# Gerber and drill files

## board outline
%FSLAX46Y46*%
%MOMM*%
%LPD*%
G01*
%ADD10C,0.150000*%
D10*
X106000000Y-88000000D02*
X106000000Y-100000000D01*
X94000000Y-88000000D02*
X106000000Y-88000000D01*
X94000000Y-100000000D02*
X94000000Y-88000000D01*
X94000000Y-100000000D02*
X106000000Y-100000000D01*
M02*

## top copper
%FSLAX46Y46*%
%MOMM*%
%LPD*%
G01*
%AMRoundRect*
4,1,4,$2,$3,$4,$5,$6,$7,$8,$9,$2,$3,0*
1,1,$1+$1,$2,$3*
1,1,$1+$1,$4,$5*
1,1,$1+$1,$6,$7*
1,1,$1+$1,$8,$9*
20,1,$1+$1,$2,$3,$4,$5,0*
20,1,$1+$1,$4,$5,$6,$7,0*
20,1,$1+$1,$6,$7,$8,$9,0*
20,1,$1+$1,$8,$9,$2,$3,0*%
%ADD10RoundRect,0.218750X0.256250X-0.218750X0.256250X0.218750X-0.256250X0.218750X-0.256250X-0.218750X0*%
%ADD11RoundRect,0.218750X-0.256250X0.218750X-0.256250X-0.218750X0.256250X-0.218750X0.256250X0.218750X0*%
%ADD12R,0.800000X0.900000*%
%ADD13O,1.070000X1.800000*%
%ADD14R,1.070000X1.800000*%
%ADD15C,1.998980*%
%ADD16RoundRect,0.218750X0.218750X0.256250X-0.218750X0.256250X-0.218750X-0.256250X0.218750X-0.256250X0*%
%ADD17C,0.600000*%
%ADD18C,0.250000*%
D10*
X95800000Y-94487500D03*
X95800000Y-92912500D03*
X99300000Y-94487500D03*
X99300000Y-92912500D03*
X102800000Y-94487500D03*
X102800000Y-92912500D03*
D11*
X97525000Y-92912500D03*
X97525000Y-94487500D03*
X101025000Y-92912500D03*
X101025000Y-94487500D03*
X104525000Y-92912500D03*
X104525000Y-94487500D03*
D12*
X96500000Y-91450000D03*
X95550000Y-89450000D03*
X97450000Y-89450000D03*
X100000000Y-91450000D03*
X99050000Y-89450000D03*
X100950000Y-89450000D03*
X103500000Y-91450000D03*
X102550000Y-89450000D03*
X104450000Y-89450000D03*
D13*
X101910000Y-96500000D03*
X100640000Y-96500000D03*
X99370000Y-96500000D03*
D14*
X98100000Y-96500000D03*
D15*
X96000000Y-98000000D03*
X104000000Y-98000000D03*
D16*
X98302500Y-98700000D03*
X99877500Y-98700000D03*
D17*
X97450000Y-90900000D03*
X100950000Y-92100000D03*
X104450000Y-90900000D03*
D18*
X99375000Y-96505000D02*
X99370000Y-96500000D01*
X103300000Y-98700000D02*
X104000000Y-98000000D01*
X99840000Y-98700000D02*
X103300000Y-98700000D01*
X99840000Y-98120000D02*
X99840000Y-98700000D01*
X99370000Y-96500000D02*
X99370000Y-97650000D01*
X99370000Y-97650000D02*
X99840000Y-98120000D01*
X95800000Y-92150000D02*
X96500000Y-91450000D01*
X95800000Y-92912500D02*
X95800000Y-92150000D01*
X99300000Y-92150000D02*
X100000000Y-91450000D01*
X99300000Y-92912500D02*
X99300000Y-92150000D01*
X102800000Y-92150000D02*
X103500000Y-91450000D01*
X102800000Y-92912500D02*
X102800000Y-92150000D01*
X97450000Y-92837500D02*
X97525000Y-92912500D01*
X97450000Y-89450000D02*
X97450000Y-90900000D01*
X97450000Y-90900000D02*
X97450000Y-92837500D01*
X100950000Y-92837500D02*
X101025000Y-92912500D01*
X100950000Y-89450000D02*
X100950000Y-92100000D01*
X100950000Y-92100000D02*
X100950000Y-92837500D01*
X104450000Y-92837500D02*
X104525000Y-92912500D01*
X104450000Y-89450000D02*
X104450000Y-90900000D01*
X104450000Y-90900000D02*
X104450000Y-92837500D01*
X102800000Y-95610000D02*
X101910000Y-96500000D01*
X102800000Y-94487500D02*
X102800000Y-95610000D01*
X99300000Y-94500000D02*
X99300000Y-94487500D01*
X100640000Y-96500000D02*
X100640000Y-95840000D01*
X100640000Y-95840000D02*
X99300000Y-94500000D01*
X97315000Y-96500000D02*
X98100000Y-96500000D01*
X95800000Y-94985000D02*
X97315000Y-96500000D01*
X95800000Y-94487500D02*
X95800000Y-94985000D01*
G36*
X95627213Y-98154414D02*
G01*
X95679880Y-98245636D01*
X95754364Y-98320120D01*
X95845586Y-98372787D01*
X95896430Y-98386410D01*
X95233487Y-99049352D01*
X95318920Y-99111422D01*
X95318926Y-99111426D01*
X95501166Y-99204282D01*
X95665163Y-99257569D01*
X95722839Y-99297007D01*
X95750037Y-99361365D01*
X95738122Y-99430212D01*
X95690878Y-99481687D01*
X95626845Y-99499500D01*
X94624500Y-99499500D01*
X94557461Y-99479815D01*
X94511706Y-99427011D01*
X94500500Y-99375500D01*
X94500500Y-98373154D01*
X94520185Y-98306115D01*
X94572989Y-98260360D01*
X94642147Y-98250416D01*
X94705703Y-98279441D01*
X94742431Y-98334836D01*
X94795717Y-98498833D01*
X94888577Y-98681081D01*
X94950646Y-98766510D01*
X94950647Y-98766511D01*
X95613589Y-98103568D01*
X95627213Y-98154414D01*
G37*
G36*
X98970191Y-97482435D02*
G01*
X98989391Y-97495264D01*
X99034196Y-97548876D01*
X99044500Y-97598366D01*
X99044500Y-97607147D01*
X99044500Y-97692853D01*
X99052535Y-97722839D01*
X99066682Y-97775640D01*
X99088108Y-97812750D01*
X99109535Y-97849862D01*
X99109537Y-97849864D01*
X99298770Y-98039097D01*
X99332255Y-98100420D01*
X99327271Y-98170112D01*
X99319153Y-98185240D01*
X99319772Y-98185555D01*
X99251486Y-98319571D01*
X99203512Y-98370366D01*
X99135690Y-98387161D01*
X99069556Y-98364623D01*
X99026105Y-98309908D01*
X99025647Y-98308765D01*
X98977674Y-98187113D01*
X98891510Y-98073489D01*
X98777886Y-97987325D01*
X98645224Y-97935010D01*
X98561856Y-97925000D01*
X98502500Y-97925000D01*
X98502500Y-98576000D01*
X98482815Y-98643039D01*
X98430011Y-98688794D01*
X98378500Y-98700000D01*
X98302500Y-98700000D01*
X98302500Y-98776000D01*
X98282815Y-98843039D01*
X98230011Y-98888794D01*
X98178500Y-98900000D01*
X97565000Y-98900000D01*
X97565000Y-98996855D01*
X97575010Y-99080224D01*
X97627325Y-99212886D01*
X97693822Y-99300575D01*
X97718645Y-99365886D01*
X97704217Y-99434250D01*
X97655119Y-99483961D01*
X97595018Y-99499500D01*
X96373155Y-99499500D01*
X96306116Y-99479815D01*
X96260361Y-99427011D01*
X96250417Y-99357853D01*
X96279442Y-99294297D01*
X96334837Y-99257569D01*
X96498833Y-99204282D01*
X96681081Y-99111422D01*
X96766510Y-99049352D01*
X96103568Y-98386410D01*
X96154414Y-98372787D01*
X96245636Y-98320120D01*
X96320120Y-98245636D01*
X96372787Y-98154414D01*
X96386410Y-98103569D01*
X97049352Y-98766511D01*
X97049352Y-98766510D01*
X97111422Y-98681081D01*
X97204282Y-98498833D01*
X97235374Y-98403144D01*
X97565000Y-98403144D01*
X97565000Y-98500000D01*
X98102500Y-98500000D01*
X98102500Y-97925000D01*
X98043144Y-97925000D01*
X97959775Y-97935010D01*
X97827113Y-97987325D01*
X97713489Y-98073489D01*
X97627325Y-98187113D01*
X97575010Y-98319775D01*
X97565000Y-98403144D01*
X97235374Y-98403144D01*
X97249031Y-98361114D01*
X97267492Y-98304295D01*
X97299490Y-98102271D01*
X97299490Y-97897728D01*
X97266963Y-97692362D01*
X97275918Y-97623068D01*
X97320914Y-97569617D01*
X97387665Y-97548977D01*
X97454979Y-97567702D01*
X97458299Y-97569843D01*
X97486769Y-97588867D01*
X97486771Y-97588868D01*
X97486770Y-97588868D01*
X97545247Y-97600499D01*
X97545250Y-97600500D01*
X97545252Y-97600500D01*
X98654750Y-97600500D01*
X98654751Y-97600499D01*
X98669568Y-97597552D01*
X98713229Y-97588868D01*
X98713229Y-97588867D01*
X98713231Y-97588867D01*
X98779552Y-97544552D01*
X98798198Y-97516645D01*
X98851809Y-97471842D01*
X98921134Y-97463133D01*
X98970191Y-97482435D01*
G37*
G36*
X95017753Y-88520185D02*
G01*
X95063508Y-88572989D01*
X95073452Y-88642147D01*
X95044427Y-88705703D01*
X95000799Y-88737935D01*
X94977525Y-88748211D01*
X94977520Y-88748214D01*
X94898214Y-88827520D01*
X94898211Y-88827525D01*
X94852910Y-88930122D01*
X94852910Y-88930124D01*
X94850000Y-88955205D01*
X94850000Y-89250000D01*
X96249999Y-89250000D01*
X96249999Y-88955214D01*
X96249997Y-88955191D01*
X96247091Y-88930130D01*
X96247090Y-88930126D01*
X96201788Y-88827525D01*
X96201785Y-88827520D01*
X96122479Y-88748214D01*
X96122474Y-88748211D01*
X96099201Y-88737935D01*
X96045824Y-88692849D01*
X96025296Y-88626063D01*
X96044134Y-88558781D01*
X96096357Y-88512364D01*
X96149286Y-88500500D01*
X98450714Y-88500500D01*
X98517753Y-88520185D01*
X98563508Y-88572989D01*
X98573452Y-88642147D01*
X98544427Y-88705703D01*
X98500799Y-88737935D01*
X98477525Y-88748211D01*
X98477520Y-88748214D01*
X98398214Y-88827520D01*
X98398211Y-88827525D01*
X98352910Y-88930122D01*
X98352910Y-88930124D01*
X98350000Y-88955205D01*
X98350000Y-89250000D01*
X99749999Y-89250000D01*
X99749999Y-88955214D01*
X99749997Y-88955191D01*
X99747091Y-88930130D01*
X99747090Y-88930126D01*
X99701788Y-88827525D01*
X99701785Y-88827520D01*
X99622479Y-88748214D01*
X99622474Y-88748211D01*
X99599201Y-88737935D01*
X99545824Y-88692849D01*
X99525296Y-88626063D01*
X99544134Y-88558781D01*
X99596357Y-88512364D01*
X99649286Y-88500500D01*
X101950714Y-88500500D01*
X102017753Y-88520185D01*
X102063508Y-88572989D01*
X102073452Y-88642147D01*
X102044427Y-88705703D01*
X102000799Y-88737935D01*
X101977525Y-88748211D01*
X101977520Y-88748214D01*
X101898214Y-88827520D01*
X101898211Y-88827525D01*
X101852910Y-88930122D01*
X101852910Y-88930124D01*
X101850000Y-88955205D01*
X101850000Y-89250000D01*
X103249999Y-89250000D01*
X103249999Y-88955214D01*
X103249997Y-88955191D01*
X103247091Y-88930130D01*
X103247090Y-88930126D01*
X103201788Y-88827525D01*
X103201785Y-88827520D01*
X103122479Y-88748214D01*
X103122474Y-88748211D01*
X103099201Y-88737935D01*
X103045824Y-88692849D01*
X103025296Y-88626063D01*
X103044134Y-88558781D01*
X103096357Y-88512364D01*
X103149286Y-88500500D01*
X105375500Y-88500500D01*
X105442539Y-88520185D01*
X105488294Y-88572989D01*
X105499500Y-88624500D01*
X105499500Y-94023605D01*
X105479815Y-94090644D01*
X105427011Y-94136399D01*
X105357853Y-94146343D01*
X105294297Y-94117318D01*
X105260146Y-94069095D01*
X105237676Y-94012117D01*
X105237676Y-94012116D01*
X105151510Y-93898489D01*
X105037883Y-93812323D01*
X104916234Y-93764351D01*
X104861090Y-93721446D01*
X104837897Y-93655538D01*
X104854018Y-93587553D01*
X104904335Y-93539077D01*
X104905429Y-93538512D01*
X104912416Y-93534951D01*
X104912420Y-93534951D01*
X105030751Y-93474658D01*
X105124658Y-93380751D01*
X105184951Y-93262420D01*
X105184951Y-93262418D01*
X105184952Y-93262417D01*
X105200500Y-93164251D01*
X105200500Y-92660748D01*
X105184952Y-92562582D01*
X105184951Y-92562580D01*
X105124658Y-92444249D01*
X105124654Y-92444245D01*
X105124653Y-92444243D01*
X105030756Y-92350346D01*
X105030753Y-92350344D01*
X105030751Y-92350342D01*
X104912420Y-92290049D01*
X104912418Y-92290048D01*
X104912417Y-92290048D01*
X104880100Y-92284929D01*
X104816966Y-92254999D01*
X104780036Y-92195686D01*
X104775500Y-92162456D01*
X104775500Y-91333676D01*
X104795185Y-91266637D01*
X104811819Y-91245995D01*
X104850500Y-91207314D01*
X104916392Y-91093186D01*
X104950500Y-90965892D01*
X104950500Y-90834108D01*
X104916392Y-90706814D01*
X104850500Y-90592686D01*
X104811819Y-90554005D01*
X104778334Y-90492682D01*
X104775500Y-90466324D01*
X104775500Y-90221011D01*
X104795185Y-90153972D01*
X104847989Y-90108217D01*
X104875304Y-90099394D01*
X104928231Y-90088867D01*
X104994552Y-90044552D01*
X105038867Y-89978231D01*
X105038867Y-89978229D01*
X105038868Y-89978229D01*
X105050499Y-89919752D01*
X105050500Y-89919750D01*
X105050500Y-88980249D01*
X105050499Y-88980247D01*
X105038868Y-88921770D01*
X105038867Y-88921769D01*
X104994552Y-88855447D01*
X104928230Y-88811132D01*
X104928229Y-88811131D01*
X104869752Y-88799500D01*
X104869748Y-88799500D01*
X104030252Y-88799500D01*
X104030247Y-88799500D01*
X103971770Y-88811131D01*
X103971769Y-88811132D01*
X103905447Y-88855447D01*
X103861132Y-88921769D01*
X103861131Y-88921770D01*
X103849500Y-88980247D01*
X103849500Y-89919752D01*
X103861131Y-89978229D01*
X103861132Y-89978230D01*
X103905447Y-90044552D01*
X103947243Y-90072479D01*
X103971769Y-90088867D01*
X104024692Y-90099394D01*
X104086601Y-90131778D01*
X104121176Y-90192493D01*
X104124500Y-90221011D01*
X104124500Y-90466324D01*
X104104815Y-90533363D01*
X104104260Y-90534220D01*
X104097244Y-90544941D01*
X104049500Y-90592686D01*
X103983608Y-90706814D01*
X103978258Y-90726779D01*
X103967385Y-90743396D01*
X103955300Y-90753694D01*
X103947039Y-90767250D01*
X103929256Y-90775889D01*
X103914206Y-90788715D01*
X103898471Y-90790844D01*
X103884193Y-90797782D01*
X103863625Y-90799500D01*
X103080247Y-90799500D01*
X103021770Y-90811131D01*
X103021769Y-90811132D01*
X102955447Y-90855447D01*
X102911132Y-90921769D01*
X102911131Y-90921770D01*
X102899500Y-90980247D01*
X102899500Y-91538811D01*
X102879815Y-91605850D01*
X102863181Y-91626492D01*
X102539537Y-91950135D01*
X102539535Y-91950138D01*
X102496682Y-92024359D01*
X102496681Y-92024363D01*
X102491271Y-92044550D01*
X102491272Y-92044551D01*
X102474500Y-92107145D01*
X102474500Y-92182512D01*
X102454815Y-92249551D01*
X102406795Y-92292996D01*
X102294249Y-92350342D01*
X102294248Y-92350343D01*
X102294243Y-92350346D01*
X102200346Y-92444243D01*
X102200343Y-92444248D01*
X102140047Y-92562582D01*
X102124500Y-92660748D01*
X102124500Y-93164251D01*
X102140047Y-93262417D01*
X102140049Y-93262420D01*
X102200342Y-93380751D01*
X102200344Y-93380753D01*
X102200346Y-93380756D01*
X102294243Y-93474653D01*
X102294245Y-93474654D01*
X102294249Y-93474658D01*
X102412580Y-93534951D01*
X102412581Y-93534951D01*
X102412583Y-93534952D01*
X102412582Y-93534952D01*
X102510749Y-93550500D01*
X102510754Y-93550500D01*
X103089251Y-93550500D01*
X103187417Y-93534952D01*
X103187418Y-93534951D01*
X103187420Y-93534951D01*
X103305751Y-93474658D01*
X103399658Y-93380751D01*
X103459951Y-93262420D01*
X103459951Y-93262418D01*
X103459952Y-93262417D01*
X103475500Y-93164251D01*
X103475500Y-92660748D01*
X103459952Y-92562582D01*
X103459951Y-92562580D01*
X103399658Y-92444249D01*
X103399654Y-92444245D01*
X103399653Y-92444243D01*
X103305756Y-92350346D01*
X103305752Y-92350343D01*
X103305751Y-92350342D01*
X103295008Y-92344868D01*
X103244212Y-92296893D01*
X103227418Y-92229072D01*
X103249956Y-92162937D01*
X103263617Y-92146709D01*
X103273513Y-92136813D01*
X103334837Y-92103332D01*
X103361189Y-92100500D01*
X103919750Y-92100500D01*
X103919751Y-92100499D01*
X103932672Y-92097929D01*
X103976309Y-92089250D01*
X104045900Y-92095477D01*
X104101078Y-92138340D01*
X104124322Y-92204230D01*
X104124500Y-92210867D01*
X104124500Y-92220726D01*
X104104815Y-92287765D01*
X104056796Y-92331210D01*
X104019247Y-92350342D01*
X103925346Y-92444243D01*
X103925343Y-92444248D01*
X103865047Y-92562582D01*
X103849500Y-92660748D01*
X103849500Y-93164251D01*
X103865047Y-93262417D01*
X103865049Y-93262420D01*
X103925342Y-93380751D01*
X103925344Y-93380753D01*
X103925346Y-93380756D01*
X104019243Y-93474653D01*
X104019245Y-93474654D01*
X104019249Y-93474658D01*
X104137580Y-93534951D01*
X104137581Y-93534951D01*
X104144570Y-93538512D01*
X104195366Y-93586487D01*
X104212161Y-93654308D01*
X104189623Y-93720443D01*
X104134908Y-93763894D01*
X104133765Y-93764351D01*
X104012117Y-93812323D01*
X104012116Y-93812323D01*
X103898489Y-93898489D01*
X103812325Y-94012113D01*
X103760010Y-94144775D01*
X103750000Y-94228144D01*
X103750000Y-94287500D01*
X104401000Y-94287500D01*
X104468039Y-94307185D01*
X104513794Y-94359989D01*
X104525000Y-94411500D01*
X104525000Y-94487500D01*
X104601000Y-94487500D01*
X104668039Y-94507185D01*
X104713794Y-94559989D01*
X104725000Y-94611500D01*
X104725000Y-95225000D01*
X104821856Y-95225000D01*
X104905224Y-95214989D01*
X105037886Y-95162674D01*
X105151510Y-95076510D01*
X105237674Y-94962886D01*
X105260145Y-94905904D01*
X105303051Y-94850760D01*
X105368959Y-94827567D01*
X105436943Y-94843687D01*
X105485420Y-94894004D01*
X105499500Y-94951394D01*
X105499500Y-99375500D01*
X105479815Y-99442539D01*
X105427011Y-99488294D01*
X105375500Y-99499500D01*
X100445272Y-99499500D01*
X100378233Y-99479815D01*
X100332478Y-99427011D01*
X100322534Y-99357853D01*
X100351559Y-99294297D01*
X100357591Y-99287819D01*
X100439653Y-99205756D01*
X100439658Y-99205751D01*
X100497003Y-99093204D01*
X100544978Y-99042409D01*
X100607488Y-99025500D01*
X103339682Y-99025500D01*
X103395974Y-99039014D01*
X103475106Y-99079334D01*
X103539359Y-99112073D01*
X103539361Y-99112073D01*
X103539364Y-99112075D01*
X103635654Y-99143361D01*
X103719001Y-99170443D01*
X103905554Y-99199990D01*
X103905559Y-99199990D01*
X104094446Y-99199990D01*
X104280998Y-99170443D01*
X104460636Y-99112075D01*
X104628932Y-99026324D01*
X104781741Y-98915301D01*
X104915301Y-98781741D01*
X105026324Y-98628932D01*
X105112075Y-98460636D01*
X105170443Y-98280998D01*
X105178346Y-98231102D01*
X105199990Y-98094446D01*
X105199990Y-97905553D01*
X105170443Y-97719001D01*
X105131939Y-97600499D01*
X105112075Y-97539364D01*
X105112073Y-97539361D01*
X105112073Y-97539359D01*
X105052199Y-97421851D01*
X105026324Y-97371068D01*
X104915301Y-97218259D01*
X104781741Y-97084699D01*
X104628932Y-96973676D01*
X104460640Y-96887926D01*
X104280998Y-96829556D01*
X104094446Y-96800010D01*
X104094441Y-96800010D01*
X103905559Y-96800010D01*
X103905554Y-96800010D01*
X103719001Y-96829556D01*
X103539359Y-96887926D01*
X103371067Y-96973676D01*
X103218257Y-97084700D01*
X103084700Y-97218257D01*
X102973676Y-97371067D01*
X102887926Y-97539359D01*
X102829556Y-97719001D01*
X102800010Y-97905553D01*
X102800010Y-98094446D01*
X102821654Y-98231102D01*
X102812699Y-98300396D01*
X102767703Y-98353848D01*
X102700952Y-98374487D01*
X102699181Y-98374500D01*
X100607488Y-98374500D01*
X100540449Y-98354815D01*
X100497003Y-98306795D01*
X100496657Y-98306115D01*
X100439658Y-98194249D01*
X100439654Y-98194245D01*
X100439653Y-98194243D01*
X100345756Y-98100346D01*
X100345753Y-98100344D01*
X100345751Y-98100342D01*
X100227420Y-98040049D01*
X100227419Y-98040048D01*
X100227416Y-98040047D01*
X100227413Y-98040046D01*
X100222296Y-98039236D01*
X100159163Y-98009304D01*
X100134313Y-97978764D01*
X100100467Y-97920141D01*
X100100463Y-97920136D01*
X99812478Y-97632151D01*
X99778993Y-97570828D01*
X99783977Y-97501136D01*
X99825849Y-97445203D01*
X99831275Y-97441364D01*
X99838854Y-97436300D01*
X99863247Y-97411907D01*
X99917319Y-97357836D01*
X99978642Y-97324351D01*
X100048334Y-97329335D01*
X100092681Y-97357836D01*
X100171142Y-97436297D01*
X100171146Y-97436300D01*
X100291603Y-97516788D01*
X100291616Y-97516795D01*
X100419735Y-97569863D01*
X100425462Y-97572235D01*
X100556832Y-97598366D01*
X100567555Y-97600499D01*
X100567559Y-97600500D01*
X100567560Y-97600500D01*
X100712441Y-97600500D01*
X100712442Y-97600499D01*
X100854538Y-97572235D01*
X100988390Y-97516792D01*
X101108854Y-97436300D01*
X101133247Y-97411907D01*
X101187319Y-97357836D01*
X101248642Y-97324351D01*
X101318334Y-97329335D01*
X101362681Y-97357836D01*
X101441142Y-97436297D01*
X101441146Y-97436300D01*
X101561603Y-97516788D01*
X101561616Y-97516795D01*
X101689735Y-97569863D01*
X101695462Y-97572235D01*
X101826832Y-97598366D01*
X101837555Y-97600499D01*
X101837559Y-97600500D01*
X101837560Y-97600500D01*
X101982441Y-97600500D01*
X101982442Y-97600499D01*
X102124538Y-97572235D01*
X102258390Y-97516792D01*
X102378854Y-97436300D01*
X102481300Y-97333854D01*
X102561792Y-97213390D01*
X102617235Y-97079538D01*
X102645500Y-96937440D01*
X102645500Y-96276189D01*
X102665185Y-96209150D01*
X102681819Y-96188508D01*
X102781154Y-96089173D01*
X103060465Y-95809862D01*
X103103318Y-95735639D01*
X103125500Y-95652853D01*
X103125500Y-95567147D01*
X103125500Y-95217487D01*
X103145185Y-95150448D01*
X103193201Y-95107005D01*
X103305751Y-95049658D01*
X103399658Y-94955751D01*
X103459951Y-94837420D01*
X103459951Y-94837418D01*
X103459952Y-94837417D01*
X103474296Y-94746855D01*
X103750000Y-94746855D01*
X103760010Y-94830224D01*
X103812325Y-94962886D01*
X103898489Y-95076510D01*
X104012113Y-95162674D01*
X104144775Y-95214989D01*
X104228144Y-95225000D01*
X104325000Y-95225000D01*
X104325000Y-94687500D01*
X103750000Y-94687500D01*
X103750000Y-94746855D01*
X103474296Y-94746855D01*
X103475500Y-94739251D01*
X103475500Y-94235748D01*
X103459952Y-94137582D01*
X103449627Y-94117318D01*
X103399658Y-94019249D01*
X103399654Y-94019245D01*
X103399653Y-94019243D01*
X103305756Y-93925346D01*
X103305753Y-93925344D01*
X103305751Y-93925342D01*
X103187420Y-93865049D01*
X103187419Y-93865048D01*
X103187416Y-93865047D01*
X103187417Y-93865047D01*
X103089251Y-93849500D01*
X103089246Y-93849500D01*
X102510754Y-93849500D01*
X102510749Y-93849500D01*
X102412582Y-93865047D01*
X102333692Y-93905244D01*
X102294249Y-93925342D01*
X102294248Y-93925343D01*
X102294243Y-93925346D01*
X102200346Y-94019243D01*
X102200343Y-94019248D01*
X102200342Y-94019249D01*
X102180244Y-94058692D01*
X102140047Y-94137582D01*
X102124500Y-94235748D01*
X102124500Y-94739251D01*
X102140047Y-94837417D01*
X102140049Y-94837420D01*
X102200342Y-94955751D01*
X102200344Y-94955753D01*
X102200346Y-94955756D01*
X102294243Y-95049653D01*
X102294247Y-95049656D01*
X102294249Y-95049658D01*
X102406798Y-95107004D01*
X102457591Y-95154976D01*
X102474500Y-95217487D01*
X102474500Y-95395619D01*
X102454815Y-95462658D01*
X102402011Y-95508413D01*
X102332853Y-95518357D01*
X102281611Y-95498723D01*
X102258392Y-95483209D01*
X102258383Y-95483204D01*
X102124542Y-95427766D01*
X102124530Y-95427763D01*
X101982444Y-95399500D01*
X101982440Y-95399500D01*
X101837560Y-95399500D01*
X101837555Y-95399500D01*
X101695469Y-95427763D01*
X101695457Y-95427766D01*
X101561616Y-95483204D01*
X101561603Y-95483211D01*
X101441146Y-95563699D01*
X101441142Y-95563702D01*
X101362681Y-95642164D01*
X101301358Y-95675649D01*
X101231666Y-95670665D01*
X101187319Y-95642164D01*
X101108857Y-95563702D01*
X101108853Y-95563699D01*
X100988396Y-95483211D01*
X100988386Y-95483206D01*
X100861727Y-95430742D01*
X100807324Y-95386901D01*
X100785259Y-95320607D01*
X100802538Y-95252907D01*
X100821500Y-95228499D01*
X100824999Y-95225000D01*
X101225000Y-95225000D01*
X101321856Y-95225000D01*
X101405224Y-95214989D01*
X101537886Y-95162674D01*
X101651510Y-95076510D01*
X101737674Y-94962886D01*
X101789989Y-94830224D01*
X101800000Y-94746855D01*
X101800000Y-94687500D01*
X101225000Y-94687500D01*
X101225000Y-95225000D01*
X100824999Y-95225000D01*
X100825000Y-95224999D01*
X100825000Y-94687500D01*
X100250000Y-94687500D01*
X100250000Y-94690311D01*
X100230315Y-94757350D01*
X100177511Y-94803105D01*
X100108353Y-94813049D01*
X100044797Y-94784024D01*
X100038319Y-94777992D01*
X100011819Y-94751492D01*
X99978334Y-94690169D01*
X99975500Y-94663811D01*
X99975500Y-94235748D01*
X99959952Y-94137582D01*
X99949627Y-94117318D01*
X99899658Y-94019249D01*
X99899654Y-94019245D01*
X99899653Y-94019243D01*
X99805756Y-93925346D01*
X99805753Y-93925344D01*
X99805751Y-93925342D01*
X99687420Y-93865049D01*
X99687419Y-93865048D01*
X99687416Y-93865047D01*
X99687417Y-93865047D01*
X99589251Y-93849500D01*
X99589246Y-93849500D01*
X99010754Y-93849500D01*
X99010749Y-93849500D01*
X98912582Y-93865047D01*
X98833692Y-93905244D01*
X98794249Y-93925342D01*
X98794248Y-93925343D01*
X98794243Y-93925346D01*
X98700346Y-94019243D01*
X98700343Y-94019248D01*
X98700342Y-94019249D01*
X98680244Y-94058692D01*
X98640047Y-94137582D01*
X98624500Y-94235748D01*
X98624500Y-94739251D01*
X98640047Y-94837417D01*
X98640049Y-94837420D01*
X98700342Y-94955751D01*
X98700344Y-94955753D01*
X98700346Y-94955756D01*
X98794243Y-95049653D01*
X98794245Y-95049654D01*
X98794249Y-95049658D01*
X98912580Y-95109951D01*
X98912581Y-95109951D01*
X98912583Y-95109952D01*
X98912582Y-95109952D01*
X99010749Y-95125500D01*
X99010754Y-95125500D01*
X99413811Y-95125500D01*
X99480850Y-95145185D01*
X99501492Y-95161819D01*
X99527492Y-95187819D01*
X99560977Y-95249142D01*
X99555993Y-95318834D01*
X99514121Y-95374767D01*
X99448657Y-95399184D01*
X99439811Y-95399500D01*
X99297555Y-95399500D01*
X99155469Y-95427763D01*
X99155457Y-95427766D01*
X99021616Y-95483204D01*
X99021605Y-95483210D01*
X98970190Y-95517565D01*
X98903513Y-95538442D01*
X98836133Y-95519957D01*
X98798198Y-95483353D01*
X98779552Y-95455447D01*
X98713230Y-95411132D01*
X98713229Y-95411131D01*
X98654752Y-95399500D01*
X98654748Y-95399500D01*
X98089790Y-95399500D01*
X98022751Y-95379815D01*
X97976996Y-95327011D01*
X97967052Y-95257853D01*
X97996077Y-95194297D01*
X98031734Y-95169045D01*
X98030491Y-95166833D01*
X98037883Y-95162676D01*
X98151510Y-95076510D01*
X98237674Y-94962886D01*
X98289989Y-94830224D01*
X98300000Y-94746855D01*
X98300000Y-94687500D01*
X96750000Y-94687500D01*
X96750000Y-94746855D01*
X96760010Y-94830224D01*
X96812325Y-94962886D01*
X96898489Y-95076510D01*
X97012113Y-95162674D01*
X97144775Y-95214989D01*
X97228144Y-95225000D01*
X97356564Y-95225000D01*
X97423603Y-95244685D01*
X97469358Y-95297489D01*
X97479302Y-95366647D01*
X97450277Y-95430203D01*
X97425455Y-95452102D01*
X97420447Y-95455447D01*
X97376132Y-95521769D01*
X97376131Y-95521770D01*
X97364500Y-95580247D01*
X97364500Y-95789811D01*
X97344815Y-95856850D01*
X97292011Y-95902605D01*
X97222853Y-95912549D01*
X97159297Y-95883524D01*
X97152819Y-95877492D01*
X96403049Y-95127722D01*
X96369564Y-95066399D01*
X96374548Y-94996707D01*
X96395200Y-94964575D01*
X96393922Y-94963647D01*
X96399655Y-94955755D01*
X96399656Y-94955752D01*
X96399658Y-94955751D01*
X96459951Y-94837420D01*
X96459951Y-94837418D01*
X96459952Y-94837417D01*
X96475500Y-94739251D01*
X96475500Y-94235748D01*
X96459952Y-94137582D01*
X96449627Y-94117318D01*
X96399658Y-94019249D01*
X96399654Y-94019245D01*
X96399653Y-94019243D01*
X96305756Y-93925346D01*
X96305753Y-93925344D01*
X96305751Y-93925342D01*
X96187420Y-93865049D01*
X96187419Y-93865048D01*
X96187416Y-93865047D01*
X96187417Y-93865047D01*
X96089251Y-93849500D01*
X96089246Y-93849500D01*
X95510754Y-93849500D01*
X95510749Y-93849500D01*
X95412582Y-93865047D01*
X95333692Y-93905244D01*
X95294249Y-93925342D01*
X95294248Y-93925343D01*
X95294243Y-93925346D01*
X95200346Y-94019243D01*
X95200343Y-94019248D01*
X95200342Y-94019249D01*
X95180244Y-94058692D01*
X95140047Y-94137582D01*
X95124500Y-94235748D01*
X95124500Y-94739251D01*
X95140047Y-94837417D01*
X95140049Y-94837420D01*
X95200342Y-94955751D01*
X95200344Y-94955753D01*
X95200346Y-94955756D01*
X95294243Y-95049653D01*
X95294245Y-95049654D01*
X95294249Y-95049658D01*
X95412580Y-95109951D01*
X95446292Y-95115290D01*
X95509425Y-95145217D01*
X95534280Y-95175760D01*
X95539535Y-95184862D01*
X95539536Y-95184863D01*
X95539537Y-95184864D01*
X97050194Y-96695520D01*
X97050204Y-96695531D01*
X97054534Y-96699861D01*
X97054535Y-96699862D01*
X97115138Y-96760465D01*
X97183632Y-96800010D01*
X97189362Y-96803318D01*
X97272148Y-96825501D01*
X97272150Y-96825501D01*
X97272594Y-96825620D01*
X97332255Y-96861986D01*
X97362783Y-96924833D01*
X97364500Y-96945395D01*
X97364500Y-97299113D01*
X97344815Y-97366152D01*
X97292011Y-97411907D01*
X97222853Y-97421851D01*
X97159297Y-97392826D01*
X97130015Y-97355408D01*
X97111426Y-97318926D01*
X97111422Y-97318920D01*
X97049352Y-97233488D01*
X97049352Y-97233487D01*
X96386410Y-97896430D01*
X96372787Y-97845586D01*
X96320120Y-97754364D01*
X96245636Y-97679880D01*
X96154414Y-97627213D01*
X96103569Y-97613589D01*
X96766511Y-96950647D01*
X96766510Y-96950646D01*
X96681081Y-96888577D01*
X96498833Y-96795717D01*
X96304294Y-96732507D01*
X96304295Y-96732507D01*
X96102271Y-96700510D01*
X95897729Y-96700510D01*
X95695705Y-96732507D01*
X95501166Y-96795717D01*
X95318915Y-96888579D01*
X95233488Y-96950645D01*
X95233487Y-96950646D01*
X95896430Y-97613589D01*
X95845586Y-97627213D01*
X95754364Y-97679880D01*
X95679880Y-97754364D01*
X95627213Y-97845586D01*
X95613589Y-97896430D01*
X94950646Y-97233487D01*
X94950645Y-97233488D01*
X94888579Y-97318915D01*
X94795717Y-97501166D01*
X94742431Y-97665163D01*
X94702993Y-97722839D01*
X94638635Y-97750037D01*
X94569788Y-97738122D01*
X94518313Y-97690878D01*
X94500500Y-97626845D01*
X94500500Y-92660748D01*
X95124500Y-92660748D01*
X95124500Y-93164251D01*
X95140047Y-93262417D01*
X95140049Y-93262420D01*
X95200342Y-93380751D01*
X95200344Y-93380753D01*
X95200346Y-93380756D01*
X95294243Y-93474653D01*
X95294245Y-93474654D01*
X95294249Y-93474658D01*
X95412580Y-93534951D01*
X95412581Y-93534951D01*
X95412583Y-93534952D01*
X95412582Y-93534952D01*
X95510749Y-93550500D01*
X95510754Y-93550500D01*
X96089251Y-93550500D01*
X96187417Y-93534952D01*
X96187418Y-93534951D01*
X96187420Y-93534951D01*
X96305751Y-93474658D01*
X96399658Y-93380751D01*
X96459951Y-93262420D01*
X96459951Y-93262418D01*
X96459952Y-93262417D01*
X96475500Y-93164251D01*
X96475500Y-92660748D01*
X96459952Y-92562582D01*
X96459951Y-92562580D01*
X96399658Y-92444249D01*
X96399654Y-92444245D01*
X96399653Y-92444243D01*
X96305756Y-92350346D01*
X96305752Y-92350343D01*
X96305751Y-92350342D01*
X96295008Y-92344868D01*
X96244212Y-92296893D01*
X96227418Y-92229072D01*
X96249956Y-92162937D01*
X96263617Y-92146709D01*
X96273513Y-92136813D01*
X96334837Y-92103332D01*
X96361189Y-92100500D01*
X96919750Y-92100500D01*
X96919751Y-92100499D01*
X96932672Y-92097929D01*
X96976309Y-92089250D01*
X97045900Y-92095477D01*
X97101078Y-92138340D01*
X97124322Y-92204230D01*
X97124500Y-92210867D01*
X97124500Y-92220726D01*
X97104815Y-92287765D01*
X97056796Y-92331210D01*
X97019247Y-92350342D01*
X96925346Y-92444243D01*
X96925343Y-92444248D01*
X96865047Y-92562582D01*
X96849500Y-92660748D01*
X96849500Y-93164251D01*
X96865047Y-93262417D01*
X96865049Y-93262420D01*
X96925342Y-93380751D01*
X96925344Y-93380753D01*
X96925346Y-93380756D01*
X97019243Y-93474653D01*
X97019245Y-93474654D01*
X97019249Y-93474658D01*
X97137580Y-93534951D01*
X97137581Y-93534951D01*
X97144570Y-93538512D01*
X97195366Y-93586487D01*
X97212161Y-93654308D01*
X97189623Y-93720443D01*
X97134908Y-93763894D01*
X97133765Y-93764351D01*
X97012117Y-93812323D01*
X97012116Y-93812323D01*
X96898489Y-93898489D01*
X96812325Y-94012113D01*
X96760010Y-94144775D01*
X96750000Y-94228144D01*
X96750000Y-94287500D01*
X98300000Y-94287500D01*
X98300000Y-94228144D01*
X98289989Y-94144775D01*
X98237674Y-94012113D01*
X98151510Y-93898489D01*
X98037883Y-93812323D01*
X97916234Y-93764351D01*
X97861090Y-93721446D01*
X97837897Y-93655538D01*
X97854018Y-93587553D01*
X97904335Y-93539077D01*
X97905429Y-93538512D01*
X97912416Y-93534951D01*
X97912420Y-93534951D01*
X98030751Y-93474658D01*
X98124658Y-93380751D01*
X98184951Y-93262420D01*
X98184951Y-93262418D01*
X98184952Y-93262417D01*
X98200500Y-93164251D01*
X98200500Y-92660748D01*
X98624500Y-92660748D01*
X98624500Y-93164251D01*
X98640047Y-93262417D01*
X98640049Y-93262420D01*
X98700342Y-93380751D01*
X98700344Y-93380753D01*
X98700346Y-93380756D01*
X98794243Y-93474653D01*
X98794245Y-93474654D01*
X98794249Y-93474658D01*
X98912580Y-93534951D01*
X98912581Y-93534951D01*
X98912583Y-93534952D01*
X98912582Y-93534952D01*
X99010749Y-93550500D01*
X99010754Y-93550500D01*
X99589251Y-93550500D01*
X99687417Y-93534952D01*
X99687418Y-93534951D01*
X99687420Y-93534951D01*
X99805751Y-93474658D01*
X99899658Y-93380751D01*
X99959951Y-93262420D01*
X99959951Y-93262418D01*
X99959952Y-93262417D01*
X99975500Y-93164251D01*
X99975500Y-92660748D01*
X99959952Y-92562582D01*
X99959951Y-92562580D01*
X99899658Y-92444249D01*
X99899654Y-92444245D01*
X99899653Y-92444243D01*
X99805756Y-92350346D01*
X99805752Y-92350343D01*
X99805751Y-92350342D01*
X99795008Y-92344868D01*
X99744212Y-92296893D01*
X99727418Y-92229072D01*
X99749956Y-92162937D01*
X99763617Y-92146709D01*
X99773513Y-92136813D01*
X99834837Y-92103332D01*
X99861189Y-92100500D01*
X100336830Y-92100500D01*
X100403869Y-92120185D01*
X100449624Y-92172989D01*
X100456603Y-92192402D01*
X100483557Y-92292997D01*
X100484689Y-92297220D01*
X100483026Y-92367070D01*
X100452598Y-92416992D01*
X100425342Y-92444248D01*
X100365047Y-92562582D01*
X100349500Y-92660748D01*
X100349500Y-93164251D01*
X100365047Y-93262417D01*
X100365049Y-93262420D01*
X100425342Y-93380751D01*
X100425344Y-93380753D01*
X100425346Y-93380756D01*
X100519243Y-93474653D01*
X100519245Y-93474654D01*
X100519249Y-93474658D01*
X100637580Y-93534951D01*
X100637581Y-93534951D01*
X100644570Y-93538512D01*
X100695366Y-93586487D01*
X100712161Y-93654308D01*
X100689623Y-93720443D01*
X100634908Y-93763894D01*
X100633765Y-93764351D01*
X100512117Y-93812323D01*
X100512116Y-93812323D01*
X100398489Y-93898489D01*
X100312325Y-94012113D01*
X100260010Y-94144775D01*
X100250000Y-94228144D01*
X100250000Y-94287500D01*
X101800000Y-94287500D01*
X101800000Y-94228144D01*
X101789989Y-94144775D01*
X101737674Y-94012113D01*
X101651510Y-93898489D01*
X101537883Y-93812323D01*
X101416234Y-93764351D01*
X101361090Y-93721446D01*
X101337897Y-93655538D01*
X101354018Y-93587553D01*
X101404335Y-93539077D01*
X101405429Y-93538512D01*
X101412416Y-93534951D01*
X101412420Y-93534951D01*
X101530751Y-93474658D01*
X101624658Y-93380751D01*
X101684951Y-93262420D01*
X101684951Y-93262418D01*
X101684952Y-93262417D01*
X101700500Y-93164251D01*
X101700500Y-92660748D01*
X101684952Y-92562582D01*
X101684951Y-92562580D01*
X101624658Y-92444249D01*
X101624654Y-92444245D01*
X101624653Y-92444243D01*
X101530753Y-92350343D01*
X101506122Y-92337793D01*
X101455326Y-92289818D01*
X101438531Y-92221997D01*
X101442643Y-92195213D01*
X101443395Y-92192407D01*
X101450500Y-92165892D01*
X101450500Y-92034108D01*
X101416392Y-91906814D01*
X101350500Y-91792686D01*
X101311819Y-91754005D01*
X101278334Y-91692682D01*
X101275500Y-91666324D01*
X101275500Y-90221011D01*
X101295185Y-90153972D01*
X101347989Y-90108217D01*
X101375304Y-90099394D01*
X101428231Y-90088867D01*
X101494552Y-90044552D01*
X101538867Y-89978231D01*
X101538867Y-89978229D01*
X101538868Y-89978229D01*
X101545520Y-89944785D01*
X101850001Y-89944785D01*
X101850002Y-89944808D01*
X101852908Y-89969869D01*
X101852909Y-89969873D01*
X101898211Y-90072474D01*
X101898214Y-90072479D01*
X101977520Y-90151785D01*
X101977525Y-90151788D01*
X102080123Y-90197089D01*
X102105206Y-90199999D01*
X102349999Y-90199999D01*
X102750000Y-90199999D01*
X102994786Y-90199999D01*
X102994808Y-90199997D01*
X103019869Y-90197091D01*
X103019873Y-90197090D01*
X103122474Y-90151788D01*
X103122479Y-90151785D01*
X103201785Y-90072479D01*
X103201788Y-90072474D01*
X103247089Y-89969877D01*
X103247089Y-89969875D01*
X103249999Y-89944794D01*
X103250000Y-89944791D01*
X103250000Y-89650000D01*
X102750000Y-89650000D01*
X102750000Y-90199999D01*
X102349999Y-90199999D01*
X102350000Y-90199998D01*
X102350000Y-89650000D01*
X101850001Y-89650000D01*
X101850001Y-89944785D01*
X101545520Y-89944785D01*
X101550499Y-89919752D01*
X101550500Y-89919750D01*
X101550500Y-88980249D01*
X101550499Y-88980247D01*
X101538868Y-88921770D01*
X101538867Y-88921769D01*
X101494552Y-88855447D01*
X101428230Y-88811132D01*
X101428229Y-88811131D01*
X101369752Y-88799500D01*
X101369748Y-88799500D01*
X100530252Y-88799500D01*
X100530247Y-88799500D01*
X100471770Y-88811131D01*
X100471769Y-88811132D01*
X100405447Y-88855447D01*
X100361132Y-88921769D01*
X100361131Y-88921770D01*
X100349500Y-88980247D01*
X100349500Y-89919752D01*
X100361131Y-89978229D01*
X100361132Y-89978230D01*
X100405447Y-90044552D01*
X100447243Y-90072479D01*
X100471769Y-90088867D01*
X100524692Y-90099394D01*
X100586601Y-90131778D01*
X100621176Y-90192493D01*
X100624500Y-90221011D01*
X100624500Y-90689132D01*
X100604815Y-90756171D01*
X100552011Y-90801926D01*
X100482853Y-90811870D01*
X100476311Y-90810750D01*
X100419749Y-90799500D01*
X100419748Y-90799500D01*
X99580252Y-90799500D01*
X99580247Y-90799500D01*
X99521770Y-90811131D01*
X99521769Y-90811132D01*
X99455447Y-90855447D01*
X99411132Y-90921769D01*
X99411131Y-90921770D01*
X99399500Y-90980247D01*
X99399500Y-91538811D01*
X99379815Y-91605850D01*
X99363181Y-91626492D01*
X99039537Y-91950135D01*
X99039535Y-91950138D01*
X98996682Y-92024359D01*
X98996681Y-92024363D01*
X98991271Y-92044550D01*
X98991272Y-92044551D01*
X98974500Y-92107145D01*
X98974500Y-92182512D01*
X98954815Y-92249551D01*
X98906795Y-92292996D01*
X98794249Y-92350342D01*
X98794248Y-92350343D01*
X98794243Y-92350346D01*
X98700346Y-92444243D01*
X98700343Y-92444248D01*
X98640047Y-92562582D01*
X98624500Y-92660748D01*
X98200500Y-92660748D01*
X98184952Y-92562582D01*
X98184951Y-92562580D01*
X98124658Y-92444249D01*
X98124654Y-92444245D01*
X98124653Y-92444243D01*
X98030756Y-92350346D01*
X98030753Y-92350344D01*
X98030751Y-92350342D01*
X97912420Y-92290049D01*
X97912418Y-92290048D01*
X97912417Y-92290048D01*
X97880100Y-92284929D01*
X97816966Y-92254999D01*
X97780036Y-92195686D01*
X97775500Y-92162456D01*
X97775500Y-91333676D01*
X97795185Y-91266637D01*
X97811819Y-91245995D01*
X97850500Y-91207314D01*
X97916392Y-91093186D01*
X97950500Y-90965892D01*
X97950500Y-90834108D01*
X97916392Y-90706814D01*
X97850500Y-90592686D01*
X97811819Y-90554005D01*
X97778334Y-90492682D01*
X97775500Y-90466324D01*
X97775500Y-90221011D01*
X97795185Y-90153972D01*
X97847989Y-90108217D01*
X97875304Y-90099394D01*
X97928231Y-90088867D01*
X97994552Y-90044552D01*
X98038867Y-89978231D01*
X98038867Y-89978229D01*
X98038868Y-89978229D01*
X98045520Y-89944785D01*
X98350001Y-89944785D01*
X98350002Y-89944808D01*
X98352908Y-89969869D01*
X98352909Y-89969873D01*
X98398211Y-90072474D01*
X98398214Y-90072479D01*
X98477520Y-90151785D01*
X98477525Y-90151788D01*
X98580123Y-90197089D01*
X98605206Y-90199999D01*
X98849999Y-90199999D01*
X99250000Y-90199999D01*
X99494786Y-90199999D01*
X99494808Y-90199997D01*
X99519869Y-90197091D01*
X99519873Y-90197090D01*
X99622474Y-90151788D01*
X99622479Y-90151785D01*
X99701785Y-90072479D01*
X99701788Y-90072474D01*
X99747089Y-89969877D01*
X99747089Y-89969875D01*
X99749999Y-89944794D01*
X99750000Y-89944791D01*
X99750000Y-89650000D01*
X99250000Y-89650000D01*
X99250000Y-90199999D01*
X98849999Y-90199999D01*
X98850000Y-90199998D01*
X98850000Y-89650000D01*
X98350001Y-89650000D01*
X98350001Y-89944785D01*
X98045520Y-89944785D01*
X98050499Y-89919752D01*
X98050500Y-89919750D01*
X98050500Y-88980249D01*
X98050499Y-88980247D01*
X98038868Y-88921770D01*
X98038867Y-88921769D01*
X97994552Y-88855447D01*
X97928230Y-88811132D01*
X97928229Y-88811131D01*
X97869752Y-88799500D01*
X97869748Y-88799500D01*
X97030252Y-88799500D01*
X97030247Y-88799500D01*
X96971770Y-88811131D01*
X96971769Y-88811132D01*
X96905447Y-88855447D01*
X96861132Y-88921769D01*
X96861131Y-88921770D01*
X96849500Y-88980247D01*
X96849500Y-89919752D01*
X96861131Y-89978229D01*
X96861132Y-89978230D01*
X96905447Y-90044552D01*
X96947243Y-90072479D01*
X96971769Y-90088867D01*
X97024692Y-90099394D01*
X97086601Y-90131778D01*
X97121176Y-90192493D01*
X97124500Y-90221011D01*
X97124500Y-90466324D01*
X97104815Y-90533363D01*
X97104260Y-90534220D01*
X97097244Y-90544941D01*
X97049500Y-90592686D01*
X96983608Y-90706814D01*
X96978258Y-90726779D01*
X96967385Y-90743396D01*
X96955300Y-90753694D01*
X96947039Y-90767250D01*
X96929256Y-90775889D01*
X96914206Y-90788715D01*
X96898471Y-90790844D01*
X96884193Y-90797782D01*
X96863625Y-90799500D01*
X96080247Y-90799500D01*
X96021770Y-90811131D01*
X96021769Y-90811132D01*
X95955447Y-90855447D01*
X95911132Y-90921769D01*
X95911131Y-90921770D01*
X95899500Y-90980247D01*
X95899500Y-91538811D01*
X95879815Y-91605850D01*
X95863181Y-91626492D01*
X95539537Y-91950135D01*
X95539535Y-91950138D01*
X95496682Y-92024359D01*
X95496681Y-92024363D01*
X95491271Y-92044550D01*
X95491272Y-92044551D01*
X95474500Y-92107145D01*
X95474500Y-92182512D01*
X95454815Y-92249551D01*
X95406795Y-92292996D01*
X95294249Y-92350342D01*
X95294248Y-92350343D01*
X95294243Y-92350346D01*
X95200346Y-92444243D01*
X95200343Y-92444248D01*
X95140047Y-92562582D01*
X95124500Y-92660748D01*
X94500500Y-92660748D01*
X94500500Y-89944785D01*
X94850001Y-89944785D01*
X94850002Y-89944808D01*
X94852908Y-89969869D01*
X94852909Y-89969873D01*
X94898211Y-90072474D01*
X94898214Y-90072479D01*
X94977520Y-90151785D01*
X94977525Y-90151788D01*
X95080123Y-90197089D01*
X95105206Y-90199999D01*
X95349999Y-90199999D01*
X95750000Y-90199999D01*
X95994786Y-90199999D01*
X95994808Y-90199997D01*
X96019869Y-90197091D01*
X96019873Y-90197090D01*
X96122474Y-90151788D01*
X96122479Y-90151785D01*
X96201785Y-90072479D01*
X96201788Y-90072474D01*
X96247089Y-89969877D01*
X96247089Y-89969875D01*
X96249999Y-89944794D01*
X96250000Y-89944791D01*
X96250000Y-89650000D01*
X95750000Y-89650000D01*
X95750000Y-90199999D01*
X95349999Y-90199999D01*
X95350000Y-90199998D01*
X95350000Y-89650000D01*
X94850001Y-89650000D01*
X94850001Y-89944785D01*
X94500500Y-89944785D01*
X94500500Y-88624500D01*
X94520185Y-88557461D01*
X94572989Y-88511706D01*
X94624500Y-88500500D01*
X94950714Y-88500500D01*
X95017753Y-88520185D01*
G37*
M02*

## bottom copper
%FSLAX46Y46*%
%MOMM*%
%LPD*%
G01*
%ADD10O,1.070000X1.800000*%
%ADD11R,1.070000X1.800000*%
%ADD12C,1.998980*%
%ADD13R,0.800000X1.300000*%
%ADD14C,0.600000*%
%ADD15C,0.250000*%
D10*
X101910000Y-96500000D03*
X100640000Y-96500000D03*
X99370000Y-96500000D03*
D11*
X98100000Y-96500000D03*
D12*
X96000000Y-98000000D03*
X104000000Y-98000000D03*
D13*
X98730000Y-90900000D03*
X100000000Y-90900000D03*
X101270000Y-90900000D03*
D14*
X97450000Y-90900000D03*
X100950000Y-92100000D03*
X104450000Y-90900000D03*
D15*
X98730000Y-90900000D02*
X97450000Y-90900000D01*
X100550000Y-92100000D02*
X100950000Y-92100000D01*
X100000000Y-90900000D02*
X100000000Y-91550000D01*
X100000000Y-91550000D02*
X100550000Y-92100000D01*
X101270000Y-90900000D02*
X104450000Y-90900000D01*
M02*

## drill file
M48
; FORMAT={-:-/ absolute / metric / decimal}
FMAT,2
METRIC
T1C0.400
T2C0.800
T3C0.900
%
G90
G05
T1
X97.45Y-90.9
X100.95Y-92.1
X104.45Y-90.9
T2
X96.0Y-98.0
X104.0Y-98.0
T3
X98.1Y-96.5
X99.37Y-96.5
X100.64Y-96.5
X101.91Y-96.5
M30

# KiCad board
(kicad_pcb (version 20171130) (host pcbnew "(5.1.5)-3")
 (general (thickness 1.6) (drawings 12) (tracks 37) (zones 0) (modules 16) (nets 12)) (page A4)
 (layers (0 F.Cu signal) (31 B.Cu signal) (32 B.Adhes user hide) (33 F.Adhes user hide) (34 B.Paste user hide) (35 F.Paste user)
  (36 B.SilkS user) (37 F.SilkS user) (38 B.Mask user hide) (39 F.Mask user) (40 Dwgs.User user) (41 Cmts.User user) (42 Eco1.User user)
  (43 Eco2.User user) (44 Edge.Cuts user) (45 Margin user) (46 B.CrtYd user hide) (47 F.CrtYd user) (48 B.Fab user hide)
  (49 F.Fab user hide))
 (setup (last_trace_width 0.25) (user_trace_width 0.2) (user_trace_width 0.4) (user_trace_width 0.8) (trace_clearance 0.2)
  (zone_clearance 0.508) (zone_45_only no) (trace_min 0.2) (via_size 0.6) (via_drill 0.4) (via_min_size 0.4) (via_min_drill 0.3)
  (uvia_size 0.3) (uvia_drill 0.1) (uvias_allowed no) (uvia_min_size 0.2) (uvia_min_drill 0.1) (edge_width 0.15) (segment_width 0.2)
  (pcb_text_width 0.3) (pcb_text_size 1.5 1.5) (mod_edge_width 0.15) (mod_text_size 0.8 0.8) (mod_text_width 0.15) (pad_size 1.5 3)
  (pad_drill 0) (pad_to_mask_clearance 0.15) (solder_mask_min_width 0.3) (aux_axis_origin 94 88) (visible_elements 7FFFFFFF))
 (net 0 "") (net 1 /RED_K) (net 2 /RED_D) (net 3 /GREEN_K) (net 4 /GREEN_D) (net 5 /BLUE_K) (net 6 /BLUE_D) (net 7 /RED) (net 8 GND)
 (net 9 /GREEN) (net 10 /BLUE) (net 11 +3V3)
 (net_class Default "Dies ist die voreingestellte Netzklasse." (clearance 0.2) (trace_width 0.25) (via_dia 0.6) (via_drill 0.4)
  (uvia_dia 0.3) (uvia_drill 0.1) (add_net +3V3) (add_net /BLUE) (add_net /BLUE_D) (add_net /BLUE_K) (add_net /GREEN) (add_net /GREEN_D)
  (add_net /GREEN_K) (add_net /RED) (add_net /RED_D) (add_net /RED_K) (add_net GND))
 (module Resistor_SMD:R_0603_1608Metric (layer F.Cu) (at 95.8 93.7 90)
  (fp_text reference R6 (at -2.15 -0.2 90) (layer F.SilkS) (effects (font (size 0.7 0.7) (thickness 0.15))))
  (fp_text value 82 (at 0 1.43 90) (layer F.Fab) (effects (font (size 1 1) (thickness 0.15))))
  (pad 1 smd roundrect (at -0.7875 0 90) (size 0.875 0.95) (layers F.Cu F.Paste F.Mask) (roundrect_rratio 0.25) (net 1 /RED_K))
  (pad 2 smd roundrect (at 0.7875 0 90) (size 0.875 0.95) (layers F.Cu F.Paste F.Mask) (roundrect_rratio 0.25) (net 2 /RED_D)))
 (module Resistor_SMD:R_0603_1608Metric (layer F.Cu) (at 99.3 93.7 90)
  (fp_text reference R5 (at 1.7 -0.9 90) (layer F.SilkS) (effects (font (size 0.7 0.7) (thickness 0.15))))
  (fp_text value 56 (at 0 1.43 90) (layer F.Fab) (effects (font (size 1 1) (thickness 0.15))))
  (pad 1 smd roundrect (at -0.7875 0 90) (size 0.875 0.95) (layers F.Cu F.Paste F.Mask) (roundrect_rratio 0.25) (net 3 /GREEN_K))
  (pad 2 smd roundrect (at 0.7875 0 90) (size 0.875 0.95) (layers F.Cu F.Paste F.Mask) (roundrect_rratio 0.25) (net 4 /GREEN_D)))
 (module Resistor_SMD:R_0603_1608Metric (layer F.Cu) (at 102.8 93.7 90)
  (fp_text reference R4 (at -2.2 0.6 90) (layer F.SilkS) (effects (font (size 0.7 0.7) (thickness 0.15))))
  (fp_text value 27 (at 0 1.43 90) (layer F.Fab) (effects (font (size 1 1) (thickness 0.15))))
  (pad 1 smd roundrect (at -0.7875 0 90) (size 0.875 0.95) (layers F.Cu F.Paste F.Mask) (roundrect_rratio 0.25) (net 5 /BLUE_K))
  (pad 2 smd roundrect (at 0.7875 0 90) (size 0.875 0.95) (layers F.Cu F.Paste F.Mask) (roundrect_rratio 0.25) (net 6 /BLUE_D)))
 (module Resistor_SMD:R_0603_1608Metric (layer F.Cu) (at 97.525 93.7 270)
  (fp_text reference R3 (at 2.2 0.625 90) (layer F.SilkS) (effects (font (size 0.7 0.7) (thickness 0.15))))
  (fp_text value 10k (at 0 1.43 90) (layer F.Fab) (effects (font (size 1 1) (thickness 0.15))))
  (pad 1 smd roundrect (at -0.7875 0 270) (size 0.875 0.95) (layers F.Cu F.Paste F.Mask) (roundrect_rratio 0.25) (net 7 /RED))
  (pad 2 smd roundrect (at 0.7875 0 270) (size 0.875 0.95) (layers F.Cu F.Paste F.Mask) (roundrect_rratio 0.25) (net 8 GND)))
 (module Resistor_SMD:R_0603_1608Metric (layer F.Cu) (at 101.025 93.7 270)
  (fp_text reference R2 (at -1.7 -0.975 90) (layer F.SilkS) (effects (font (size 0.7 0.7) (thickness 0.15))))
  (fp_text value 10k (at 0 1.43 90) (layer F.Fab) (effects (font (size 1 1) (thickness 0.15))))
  (pad 1 smd roundrect (at -0.7875 0 270) (size 0.875 0.95) (layers F.Cu F.Paste F.Mask) (roundrect_rratio 0.25) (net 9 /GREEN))
  (pad 2 smd roundrect (at 0.7875 0 270) (size 0.875 0.95) (layers F.Cu F.Paste F.Mask) (roundrect_rratio 0.25) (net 8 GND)))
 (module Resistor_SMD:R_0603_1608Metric (layer F.Cu) (at 104.525 93.7 270)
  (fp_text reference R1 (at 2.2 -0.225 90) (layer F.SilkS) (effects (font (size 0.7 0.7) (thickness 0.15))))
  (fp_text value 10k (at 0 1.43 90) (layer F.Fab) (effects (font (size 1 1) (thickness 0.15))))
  (pad 1 smd roundrect (at -0.7875 0 270) (size 0.875 0.95) (layers F.Cu F.Paste F.Mask) (roundrect_rratio 0.25) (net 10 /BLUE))
  (pad 2 smd roundrect (at 0.7875 0 270) (size 0.875 0.95) (layers F.Cu F.Paste F.Mask) (roundrect_rratio 0.25) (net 8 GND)))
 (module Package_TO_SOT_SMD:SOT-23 (layer F.Cu) (at 96.5 90.45 270)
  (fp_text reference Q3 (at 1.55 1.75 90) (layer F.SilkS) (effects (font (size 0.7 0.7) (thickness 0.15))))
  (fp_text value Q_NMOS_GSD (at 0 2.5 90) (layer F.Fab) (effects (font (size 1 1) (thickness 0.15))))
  (pad 3 smd rect (at 1 0 270) (size 0.9 0.8) (layers F.Cu F.Paste F.Mask) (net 2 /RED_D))
  (pad 2 smd rect (at -1 0.95 270) (size 0.9 0.8) (layers F.Cu F.Paste F.Mask) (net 8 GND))
  (pad 1 smd rect (at -1 -0.95 270) (size 0.9 0.8) (layers F.Cu F.Paste F.Mask) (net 7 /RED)))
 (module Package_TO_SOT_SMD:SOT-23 (layer F.Cu) (at 100 90.45 270)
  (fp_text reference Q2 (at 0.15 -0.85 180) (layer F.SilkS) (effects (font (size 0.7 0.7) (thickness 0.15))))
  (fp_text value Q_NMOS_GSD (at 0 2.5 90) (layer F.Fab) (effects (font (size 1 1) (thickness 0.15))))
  (pad 3 smd rect (at 1 0 270) (size 0.9 0.8) (layers F.Cu F.Paste F.Mask) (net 4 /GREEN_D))
  (pad 2 smd rect (at -1 0.95 270) (size 0.9 0.8) (layers F.Cu F.Paste F.Mask) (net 8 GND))
  (pad 1 smd rect (at -1 -0.95 270) (size 0.9 0.8) (layers F.Cu F.Paste F.Mask) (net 9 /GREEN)))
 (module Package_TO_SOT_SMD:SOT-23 (layer F.Cu) (at 103.5 90.45 270)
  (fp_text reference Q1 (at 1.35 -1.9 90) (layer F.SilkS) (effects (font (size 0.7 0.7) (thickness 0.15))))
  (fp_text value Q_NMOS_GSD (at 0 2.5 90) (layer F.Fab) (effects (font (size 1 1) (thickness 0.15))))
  (pad 3 smd rect (at 1 0 270) (size 0.9 0.8) (layers F.Cu F.Paste F.Mask) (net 6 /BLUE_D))
  (pad 2 smd rect (at -1 0.95 270) (size 0.9 0.8) (layers F.Cu F.Paste F.Mask) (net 8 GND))
  (pad 1 smd rect (at -1 -0.95 270) (size 0.9 0.8) (layers F.Cu F.Paste F.Mask) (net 10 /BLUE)))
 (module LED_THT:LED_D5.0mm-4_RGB (layer F.Cu) (at 98.1 96.5)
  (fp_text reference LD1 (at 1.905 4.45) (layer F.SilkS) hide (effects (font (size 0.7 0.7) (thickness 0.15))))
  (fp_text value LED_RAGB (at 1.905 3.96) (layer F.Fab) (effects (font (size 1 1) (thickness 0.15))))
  (pad 4 thru_hole oval (at 3.81 0) (size 1.07 1.8) (drill 0.9) (layers *.Cu *.Mask) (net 5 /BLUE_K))
  (pad 3 thru_hole oval (at 2.54 0) (size 1.07 1.8) (drill 0.9) (layers *.Cu *.Mask) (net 3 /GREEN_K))
  (pad 2 thru_hole oval (at 1.27 0) (size 1.07 1.8) (drill 0.9) (layers *.Cu *.Mask) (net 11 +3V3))
  (pad 1 thru_hole rect (at 0 0) (size 1.07 1.8) (drill 0.9) (layers *.Cu *.Mask) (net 1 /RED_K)))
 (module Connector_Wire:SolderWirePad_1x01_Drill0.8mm (layer F.Cu) (at 96 98)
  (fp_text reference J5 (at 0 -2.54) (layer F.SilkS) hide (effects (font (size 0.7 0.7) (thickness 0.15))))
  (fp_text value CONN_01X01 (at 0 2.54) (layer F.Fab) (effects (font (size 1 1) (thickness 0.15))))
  (pad 1 thru_hole circle (at 0 0) (size 1.99898 1.99898) (drill 0.8001) (layers *.Cu *.Mask) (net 8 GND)))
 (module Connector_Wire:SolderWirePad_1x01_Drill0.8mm (layer F.Cu) (at 104 98)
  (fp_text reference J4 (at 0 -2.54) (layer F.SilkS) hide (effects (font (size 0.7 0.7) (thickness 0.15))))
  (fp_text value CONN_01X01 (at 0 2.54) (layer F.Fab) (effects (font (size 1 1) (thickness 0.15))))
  (pad 1 thru_hole circle (at 0 0) (size 1.99898 1.99898) (drill 0.8001) (layers *.Cu *.Mask) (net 11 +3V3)))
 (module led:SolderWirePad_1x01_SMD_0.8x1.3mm (layer B.Cu) (at 98.73 90.9)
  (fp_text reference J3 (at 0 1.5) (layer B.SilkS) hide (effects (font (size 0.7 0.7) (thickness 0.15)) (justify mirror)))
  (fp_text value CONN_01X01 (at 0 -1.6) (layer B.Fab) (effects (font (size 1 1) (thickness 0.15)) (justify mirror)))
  (pad 1 smd rect (at 0 0) (size 0.8 1.3) (layers B.Cu B.Paste B.Mask) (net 7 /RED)))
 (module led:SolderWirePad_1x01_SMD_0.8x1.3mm (layer B.Cu) (at 100 90.9)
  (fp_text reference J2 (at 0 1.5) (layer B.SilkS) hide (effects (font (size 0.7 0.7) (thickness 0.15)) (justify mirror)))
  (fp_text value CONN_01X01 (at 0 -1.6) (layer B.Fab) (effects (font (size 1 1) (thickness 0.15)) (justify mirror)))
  (pad 1 smd rect (at 0 0) (size 0.8 1.3) (layers B.Cu B.Paste B.Mask) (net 9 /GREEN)))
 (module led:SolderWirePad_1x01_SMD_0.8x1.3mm (layer B.Cu) (at 101.27 90.9)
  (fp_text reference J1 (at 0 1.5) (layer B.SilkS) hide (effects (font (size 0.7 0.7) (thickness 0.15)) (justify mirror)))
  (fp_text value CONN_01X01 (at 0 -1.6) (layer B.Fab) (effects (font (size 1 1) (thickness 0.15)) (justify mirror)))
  (pad 1 smd rect (at 0 0) (size 0.8 1.3) (layers B.Cu B.Paste B.Mask) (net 10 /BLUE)))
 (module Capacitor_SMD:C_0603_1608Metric (layer F.Cu) (at 99.09 98.7 180)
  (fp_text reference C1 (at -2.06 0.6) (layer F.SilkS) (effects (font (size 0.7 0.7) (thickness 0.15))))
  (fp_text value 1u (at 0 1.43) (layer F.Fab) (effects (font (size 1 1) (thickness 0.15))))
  (pad 2 smd roundrect (at 0.7875 0 180) (size 0.875 0.95) (layers F.Cu F.Paste F.Mask) (roundrect_rratio 0.25) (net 8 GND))
  (pad 1 smd roundrect (at -0.7875 0 180) (size 0.875 0.95) (layers F.Cu F.Paste F.Mask) (roundrect_rratio 0.25) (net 11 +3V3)))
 (gr_line (start 106 88) (end 106 100) (layer Edge.Cuts) (width 0.15))
 (gr_line (start 94 88) (end 106 88) (layer Edge.Cuts) (width 0.15))
 (gr_line (start 94 100) (end 94 88) (layer Edge.Cuts) (width 0.15))
 (gr_line (start 94 100) (end 106 100) (layer Edge.Cuts) (width 0.15))
 (segment (start 99.375 96.505) (end 99.37 96.5) (width 0.25) (layer F.Cu) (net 11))
 (segment (start 103.3 98.7) (end 104 98) (width 0.25) (layer F.Cu) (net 11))
 (segment (start 99.84 98.7) (end 103.3 98.7) (width 0.25) (layer F.Cu) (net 11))
 (segment (start 99.84 98.12) (end 99.84 98.7) (width 0.25) (layer F.Cu) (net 11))
 (segment (start 99.37 96.5) (end 99.37 97.65) (width 0.25) (layer F.Cu) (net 11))
 (segment (start 99.37 97.65) (end 99.84 98.12) (width 0.25) (layer F.Cu) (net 11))
 (segment (start 95.8 92.15) (end 96.5 91.45) (width 0.25) (layer F.Cu) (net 2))
 (segment (start 95.8 92.9125) (end 95.8 92.15) (width 0.25) (layer F.Cu) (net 2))
 (segment (start 99.3 92.15) (end 100 91.45) (width 0.25) (layer F.Cu) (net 4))
 (segment (start 99.3 92.9125) (end 99.3 92.15) (width 0.25) (layer F.Cu) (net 4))
 (segment (start 102.8 92.15) (end 103.5 91.45) (width 0.25) (layer F.Cu) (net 6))
 (segment (start 102.8 92.9125) (end 102.8 92.15) (width 0.25) (layer F.Cu) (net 6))
 (segment (start 97.45 92.8375) (end 97.525 92.9125) (width 0.25) (layer F.Cu) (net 7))
 (segment (start 98.73 90.9) (end 97.45 90.9) (width 0.25) (layer B.Cu) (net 7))
 (segment (start 97.45 89.45) (end 97.45 90.9) (width 0.25) (layer F.Cu) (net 7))
 (via (at 97.45 90.9) (size 0.6) (drill 0.4) (layers F.Cu B.Cu) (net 7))
 (segment (start 97.45 90.9) (end 97.45 92.8375) (width 0.25) (layer F.Cu) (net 7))
 (segment (start 100.95 92.8375) (end 101.025 92.9125) (width 0.25) (layer F.Cu) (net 9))
 (via (at 100.95 92.1) (size 0.6) (drill 0.4) (layers F.Cu B.Cu) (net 9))
 (segment (start 100.95 89.45) (end 100.95 92.1) (width 0.25) (layer F.Cu) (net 9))
 (segment (start 100.95 92.1) (end 100.95 92.8375) (width 0.25) (layer F.Cu) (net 9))
 (segment (start 100.55 92.1) (end 100.95 92.1) (width 0.25) (layer B.Cu) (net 9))
 (segment (start 100 90.9) (end 100 91.55) (width 0.25) (layer B.Cu) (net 9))
 (segment (start 100 91.55) (end 100.55 92.1) (width 0.25) (layer B.Cu) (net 9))
 (segment (start 104.45 92.8375) (end 104.525 92.9125) (width 0.25) (layer F.Cu) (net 10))
 (via (at 104.45 90.9) (size 0.6) (drill 0.4) (layers F.Cu B.Cu) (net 10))
 (segment (start 101.27 90.9) (end 104.45 90.9) (width 0.25) (layer B.Cu) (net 10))
 (segment (start 104.45 89.45) (end 104.45 90.9) (width 0.25) (layer F.Cu) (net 10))
 (segment (start 104.45 90.9) (end 104.45 92.8375) (width 0.25) (layer F.Cu) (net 10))
 (segment (start 102.8 95.61) (end 101.91 96.5) (width 0.25) (layer F.Cu) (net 5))
 (segment (start 102.8 94.4875) (end 102.8 95.61) (width 0.25) (layer F.Cu) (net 5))
 (segment (start 99.3 94.5) (end 99.3 94.4875) (width 0.25) (layer F.Cu) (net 3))
 (segment (start 100.64 96.5) (end 100.64 95.84) (width 0.25) (layer F.Cu) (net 3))
 (segment (start 100.64 95.84) (end 99.3 94.5) (width 0.25) (layer F.Cu) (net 3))
 (segment (start 97.315 96.5) (end 98.1 96.5) (width 0.25) (layer F.Cu) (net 1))
 (segment (start 95.8 94.985) (end 97.315 96.5) (width 0.25) (layer F.Cu) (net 1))
 (segment (start 95.8 94.4875) (end 95.8 94.985) (width 0.25) (layer F.Cu) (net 1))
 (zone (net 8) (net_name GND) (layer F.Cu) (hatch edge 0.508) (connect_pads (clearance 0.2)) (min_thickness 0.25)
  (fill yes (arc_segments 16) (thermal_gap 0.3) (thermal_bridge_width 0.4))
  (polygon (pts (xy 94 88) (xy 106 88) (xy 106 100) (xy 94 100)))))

